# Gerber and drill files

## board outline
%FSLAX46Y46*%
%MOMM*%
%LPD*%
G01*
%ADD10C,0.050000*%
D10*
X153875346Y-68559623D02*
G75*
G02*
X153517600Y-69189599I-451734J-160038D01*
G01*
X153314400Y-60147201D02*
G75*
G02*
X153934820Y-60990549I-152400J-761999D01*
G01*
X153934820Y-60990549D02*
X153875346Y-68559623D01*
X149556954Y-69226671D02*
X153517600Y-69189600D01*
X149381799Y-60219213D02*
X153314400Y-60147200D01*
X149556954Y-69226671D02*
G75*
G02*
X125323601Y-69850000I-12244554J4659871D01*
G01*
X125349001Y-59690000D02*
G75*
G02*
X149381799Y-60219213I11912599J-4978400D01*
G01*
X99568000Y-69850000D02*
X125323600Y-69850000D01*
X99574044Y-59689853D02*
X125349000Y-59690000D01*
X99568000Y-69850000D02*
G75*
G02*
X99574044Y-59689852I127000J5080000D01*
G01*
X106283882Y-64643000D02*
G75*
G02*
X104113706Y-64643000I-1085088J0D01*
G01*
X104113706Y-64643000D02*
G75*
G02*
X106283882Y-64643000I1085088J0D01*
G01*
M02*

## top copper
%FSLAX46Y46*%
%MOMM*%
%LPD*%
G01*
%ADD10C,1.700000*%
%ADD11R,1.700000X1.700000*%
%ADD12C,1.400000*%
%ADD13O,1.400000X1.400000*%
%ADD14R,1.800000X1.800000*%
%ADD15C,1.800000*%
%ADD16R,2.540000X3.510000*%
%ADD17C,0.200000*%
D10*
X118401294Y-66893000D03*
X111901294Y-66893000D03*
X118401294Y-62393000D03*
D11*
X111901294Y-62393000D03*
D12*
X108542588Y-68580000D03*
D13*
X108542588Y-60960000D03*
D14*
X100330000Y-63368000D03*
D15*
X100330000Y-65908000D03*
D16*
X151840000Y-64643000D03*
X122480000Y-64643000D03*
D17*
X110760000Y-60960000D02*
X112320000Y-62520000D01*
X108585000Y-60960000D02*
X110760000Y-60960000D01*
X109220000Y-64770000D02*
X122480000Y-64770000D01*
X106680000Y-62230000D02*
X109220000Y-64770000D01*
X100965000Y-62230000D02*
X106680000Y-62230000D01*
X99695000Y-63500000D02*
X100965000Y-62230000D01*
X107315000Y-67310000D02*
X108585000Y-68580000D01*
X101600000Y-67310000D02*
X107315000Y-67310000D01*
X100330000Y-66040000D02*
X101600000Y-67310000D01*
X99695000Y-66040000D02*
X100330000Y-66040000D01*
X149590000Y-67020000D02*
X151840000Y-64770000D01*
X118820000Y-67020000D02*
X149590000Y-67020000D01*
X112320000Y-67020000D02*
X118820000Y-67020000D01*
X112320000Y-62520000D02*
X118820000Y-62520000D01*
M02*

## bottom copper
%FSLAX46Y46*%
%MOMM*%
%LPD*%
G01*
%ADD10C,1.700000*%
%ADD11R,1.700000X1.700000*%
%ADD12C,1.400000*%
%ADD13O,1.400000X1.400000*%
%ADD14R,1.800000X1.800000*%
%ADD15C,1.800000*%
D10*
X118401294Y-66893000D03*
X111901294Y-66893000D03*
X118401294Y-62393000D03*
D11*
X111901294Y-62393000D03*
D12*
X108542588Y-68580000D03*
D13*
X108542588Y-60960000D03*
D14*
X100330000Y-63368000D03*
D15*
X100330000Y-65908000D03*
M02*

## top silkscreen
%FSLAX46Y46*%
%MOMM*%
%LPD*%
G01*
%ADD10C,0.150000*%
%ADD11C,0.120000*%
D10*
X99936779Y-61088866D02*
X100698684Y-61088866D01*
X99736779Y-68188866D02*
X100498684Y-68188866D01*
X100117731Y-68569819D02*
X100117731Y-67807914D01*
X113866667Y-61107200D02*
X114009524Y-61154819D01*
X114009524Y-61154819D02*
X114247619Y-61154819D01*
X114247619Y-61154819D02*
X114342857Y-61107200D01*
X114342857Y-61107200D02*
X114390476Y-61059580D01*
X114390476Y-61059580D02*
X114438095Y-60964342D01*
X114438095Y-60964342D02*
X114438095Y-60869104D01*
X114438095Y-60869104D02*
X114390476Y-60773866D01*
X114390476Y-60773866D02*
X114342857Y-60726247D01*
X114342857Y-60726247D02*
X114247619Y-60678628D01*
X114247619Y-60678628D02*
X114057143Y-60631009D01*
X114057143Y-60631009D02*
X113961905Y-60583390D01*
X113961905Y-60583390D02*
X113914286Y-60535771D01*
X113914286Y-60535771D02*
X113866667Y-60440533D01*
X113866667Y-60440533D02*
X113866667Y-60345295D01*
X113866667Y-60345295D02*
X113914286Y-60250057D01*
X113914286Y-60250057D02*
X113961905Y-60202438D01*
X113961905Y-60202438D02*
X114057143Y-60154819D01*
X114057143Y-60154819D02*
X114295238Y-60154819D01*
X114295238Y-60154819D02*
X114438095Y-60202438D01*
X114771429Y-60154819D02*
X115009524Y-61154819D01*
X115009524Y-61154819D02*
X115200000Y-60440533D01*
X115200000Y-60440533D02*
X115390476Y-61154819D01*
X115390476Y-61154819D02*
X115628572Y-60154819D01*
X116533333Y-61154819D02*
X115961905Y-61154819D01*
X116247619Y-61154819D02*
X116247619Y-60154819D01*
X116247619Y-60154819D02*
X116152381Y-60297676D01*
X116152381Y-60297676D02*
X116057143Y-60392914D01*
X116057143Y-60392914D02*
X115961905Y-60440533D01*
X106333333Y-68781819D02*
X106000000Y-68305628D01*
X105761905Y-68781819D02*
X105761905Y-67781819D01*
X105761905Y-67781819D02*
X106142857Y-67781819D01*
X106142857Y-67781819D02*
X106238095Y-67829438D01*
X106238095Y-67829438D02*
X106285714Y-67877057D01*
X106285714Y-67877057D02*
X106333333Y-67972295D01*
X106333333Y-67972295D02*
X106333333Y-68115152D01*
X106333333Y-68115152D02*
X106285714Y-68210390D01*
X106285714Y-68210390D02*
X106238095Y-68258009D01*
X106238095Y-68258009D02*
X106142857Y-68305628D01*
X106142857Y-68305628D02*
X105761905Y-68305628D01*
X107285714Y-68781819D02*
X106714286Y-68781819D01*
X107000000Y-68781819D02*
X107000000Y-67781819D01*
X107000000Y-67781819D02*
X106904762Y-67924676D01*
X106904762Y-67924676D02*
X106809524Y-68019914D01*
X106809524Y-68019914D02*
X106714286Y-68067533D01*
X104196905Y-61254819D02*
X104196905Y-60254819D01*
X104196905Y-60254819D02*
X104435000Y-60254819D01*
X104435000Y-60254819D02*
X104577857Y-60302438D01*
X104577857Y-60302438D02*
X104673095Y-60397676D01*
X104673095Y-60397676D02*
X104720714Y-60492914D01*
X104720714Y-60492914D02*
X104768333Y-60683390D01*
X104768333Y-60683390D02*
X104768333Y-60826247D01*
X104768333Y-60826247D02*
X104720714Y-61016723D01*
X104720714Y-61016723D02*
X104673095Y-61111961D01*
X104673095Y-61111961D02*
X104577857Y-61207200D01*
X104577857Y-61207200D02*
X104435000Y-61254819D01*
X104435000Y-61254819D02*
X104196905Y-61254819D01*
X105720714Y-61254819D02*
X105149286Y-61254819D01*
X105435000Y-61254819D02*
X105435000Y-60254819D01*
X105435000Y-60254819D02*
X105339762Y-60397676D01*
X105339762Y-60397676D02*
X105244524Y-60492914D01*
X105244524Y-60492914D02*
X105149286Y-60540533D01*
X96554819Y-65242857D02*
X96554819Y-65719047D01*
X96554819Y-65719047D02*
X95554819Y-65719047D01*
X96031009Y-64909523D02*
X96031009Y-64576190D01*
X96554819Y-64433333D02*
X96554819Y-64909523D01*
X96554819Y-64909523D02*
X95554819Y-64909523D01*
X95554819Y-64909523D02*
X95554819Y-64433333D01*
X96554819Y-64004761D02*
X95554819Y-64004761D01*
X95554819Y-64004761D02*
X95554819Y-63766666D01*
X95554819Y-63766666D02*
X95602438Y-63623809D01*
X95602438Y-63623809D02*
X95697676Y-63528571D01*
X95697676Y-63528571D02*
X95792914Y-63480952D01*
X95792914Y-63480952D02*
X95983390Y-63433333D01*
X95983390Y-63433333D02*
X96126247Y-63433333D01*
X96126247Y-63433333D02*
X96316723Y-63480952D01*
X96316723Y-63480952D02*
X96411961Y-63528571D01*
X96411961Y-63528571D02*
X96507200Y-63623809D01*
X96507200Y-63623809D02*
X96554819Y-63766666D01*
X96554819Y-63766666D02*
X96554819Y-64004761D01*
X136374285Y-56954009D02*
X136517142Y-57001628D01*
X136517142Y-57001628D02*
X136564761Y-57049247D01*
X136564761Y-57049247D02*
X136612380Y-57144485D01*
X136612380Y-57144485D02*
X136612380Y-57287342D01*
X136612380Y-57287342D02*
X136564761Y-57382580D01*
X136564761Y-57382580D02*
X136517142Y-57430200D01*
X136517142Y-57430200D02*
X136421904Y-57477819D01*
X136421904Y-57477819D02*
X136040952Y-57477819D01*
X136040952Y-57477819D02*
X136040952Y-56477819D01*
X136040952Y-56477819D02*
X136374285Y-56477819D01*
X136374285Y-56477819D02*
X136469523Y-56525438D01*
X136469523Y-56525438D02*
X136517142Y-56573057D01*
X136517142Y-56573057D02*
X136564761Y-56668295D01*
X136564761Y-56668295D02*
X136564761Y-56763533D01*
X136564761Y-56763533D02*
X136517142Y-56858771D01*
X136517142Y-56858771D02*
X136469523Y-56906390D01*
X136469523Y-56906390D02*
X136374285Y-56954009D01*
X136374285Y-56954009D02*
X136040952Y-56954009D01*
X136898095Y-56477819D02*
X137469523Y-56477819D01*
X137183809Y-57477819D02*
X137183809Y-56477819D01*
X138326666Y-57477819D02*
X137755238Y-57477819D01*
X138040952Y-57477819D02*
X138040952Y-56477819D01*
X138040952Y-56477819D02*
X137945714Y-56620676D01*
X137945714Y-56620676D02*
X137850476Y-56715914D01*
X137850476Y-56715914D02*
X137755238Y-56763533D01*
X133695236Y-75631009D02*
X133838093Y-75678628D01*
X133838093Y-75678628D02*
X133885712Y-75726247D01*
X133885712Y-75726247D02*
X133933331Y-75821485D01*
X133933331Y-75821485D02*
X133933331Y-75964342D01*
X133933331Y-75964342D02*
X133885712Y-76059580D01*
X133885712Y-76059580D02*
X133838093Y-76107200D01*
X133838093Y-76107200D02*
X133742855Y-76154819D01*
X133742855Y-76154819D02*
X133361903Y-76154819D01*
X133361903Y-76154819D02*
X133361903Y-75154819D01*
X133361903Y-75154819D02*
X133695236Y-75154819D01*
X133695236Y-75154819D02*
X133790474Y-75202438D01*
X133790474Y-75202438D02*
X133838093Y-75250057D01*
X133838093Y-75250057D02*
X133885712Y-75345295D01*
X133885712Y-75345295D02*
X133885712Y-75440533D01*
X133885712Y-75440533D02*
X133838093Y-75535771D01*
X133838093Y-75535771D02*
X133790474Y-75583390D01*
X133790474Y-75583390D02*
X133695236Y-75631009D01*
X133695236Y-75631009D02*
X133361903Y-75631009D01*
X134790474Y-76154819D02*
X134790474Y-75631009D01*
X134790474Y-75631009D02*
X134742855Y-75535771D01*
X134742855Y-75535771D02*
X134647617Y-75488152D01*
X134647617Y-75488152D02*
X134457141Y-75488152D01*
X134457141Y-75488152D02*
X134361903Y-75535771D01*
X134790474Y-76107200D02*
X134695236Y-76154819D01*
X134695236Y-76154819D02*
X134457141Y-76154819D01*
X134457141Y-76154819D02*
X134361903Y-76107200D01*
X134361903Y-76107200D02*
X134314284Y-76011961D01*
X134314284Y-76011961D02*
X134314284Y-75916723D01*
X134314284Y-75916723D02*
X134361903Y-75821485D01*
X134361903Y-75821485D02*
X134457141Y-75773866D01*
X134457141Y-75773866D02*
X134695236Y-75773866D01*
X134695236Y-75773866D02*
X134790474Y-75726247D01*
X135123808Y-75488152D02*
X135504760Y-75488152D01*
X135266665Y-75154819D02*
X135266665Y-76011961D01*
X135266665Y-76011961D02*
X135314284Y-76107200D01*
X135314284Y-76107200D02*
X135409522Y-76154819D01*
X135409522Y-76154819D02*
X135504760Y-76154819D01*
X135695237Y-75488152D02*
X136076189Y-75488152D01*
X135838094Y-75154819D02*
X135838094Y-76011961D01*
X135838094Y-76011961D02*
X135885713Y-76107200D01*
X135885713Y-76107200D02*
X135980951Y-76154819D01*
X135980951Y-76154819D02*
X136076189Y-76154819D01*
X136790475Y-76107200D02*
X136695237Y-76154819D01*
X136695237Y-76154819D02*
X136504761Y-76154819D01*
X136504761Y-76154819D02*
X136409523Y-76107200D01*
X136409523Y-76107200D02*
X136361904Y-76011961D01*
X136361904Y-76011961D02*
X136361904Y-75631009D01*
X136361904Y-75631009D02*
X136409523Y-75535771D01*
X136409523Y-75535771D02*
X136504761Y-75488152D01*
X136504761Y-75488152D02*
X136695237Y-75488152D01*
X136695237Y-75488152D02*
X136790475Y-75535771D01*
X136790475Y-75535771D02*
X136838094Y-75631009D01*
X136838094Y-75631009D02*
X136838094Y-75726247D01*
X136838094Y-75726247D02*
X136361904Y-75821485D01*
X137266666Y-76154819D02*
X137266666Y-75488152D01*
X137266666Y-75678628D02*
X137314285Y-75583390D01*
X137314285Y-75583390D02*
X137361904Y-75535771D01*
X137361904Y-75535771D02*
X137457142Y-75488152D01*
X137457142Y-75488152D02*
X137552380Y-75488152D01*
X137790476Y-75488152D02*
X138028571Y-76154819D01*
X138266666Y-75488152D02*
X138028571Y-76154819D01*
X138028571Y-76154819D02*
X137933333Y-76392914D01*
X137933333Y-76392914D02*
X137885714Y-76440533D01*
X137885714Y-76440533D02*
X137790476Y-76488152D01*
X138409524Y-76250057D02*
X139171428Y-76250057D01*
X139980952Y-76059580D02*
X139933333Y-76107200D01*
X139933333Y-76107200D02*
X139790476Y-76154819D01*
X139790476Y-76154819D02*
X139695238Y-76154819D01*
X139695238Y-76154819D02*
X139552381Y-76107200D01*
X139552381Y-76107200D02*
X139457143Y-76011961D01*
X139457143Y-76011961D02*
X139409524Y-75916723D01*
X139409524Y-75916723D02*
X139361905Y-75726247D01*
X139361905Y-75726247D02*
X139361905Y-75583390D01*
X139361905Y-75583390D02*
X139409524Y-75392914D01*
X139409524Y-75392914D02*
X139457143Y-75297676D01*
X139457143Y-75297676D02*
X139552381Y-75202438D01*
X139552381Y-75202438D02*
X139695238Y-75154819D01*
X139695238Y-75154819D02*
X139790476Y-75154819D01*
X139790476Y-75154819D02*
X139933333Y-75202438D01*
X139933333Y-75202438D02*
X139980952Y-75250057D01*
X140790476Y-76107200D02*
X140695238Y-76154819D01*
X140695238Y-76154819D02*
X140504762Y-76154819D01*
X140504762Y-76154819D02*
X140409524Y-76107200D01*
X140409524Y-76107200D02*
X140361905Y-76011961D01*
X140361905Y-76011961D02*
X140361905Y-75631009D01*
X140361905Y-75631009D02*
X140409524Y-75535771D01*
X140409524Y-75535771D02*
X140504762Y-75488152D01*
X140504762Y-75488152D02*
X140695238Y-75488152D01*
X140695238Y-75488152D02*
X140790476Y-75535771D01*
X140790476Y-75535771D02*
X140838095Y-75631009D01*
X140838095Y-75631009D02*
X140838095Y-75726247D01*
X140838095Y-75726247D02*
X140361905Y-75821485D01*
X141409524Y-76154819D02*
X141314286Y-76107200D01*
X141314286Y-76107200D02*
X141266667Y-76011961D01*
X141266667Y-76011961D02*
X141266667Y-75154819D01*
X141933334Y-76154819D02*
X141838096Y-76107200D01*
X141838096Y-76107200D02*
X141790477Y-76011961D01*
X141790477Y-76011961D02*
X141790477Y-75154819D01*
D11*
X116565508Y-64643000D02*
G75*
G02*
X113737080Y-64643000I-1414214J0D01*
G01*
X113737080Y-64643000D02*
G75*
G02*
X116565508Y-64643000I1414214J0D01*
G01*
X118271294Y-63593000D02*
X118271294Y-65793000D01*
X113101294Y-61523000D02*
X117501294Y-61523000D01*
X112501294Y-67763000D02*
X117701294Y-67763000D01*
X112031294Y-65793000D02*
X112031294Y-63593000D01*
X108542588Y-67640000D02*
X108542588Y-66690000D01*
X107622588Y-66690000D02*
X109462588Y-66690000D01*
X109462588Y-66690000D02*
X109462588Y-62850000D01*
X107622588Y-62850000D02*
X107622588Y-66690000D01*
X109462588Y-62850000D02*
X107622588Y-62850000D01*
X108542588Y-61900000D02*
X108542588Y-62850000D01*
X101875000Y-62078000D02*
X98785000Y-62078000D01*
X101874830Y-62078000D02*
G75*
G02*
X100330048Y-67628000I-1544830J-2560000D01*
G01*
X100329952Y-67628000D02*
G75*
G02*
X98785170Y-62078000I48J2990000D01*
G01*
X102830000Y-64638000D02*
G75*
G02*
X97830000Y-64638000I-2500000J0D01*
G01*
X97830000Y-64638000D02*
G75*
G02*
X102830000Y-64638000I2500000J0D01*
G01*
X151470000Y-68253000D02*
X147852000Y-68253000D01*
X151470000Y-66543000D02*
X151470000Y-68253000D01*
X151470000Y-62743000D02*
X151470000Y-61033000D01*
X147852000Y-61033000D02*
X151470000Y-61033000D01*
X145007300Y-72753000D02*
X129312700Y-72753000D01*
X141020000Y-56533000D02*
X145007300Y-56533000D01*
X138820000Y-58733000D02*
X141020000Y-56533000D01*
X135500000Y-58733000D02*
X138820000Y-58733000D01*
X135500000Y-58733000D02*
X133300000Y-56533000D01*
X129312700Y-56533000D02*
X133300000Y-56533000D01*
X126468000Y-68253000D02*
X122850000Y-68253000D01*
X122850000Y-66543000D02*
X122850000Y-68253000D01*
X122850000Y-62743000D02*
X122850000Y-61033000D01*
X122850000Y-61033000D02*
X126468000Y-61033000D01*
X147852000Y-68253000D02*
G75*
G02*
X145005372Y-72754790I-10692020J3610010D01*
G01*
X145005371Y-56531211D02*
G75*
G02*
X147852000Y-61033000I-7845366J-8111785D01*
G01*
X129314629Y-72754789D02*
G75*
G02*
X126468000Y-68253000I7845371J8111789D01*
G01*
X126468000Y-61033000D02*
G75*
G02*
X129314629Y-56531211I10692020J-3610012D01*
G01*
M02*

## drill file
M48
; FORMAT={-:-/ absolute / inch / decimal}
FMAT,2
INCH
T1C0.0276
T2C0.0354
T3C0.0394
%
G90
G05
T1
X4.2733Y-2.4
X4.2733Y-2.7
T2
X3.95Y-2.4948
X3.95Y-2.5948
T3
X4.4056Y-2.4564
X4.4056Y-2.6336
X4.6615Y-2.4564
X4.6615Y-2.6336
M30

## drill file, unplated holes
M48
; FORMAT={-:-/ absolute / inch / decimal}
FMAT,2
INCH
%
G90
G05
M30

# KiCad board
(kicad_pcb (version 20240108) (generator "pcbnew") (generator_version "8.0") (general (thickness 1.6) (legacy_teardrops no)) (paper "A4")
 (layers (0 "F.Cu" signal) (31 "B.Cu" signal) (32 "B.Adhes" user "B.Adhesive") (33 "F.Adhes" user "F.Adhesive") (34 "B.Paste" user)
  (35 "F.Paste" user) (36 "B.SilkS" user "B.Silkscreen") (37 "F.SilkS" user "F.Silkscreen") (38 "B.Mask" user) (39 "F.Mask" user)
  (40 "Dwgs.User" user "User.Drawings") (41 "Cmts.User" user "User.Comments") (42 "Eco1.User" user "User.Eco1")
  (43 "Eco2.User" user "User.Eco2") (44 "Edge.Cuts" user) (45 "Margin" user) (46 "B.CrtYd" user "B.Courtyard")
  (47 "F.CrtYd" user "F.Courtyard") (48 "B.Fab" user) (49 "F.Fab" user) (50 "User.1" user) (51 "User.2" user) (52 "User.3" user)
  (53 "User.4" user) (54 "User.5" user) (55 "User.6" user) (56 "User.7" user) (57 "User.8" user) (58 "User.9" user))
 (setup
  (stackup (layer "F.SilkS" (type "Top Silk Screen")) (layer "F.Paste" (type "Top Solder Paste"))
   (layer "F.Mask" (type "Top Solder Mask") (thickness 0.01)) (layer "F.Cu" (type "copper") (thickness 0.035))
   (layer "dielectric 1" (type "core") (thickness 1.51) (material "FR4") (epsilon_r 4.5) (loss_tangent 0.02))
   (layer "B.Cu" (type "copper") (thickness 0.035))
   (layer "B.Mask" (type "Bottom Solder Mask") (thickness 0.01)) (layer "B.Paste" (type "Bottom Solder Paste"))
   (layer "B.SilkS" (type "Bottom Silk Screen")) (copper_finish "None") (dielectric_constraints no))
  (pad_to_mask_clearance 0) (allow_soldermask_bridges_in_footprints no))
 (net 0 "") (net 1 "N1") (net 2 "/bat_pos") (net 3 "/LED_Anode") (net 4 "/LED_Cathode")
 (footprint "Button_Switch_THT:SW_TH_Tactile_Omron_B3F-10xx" (layer "F.Cu") (at 111.901294 62.393)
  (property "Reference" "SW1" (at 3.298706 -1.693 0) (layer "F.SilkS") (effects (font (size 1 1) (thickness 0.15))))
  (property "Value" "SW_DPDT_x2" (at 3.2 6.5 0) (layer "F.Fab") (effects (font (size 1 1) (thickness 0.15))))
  (fp_line (start 0.13 3.4) (end 0.13 1.2) (stroke (width 0.12) (type solid)) (layer "F.SilkS"))
  (fp_line (start 0.6 5.37) (end 5.8 5.37) (stroke (width 0.12) (type solid)) (layer "F.SilkS"))
  (fp_line (start 1.2 -0.87) (end 5.6 -0.87) (stroke (width 0.12) (type solid)) (layer "F.SilkS"))
  (fp_line (start 6.37 1.2) (end 6.37 3.4) (stroke (width 0.12) (type solid)) (layer "F.SilkS"))
  (fp_circle (center 3.25 2.25) (end 4.25 3.25) (stroke (width 0.12) (type solid)) (fill none) (layer "F.SilkS"))
  (pad "1" thru_hole rect (at 0 0) (size 1.7 1.7) (drill 1) (layers "*.Cu" "*.Mask") (remove_unused_layers no) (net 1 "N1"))
  (pad "1" thru_hole circle (at 6.5 0) (size 1.7 1.7) (drill 1) (layers "*.Cu" "*.Mask") (remove_unused_layers no) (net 1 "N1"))
  (pad "2" thru_hole circle (at 0 4.5) (size 1.7 1.7) (drill 1) (layers "*.Cu" "*.Mask") (remove_unused_layers no) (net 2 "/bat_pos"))
  (pad "2" thru_hole circle (at 6.5 4.5) (size 1.7 1.7) (drill 1) (layers "*.Cu" "*.Mask") (remove_unused_layers no) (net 2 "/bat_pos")))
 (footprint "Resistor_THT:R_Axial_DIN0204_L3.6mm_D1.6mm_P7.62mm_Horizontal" (layer "F.Cu") (at 108.542588 68.58 90)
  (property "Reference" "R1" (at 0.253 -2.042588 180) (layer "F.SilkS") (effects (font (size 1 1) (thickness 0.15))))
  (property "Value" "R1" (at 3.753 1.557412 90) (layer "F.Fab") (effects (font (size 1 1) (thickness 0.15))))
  (fp_line (start 5.73 -0.92) (end 1.89 -0.92) (stroke (width 0.12) (type solid)) (layer "F.SilkS"))
  (fp_line (start 1.89 -0.92) (end 1.89 0.92) (stroke (width 0.12) (type solid)) (layer "F.SilkS"))
  (fp_line (start 6.68 0) (end 5.73 0) (stroke (width 0.12) (type solid)) (layer "F.SilkS"))
  (fp_line (start 0.94 0) (end 1.89 0) (stroke (width 0.12) (type solid)) (layer "F.SilkS"))
  (fp_line (start 5.73 0.92) (end 5.73 -0.92) (stroke (width 0.12) (type solid)) (layer "F.SilkS"))
  (fp_line (start 1.89 0.92) (end 5.73 0.92) (stroke (width 0.12) (type solid)) (layer "F.SilkS"))
  (pad "1" thru_hole circle (at 0 0 90) (size 1.4 1.4) (drill 0.7) (layers "*.Cu" "*.Mask") (remove_unused_layers no) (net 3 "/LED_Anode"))
  (pad "2" thru_hole oval (at 7.62 0 90) (size 1.4 1.4) (drill 0.7) (layers "*.Cu" "*.Mask") (remove_unused_layers no) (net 1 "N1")))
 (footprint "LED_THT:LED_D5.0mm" (layer "F.Cu") (at 100.33 63.368 -90)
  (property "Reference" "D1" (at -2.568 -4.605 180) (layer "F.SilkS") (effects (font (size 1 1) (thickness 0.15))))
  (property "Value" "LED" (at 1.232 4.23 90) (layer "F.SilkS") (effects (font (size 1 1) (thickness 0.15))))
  (fp_line (start -1.29 -1.545) (end -1.29 1.545) (stroke (width 0.12) (type solid)) (layer "F.SilkS"))
  (fp_arc (start 4.26 0.000048) (mid 2.071756 2.880501) (end -1.29 1.54483) (stroke (width 0.12) (type solid)) (layer "F.SilkS"))
  (fp_arc (start -1.29 -1.54483) (mid 2.071756 -2.880501) (end 4.26 -0.000048) (stroke (width 0.12) (type solid)) (layer "F.SilkS"))
  (fp_circle (center 1.27 0) (end 3.77 0) (stroke (width 0.12) (type solid)) (fill none) (layer "F.SilkS"))
  (pad "1" thru_hole rect (at 0 0 270) (size 1.8 1.8) (drill 0.9) (layers "*.Cu" "*.Mask") (remove_unused_layers no) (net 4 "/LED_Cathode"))
  (pad "2" thru_hole circle (at 2.54 0 270) (size 1.8 1.8) (drill 0.9) (layers "*.Cu" "*.Mask") (remove_unused_layers no)
   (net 3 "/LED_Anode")))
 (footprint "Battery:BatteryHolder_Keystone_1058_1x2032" (layer "F.Cu") (at 137.16 64.643 180)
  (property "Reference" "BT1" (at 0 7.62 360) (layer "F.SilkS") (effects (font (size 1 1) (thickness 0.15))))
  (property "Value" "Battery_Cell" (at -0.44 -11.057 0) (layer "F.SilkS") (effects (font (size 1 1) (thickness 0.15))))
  (fp_line (start 14.31 3.61) (end 10.692 3.61) (stroke (width 0.12) (type solid)) (layer "F.SilkS"))
  (fp_line (start 14.31 1.9) (end 14.31 3.61) (stroke (width 0.12) (type solid)) (layer "F.SilkS"))
  (fp_line (start 14.31 -1.9) (end 14.31 -3.61) (stroke (width 0.12) (type solid)) (layer "F.SilkS"))
  (fp_line (start 10.692 -3.61) (end 14.31 -3.61) (stroke (width 0.12) (type solid)) (layer "F.SilkS"))
  (fp_line (start 7.8473 8.11) (end 3.86 8.11) (stroke (width 0.12) (type solid)) (layer "F.SilkS"))
  (fp_line (start 1.66 5.91) (end 3.86 8.11) (stroke (width 0.12) (type solid)) (layer "F.SilkS"))
  (fp_line (start 1.66 5.91) (end -1.66 5.91) (stroke (width 0.12) (type solid)) (layer "F.SilkS"))
  (fp_line (start -1.66 5.91) (end -3.86 8.11) (stroke (width 0.12) (type solid)) (layer "F.SilkS"))
  (fp_line (start -3.86 8.11) (end -7.8473 8.11) (stroke (width 0.12) (type solid)) (layer "F.SilkS"))
  (fp_line (start -7.8473 -8.11) (end 7.8473 -8.11) (stroke (width 0.12) (type solid)) (layer "F.SilkS"))
  (fp_line (start -10.692 3.61) (end -14.31 3.61) (stroke (width 0.12) (type solid)) (layer "F.SilkS"))
  (fp_line (start -14.31 1.9) (end -14.31 3.61) (stroke (width 0.12) (type solid)) (layer "F.SilkS"))
  (fp_line (start -14.31 -1.9) (end -14.31 -3.61) (stroke (width 0.12) (type solid)) (layer "F.SilkS"))
  (fp_line (start -14.31 -3.61) (end -10.692 -3.61) (stroke (width 0.12) (type solid)) (layer "F.SilkS"))
  (fp_arc (start 10.692 3.61) (mid 9.538084 6.031244) (end 7.845371 8.111789) (stroke (width 0.12) (type solid)) (layer "F.SilkS"))
  (fp_arc (start 7.845371 -8.111789) (mid 9.538085 -6.031244) (end 10.692 -3.61) (stroke (width 0.12) (type solid)) (layer "F.SilkS"))
  (fp_arc (start -7.845371 8.111789) (mid -9.538085 6.031244) (end -10.692 3.61) (stroke (width 0.12) (type solid)) (layer "F.SilkS"))
  (fp_arc (start -10.692 -3.61) (mid -9.538084 -6.031244) (end -7.845371 -8.111789) (stroke (width 0.12) (type solid)) (layer "F.SilkS"))
  (pad "1" smd rect (at -14.68 0 180) (size 2.54 3.51) (layers "F.Cu" "F.Paste" "F.Mask") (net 2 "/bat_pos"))
  (pad "2" smd rect (at 14.68 0 180) (size 2.54 3.51) (layers "F.Cu" "F.Paste" "F.Mask") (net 4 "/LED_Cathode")))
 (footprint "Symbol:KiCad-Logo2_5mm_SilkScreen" (layer "B.Cu") (at 136.8806 62.0268 180)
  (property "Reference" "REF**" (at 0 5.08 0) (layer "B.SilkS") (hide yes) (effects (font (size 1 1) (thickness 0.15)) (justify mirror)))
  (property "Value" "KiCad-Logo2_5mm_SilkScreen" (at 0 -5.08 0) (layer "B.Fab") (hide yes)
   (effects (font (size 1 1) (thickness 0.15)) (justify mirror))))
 (gr_line (start 99.568 69.85) (end 125.3236 69.85) (locked yes) (stroke (width 0.05) (type default)) (layer "Edge.Cuts"))
 (gr_line (start 99.574044 59.689853) (end 125.349 59.69) (locked yes) (stroke (width 0.05) (type default)) (layer "Edge.Cuts"))
 (gr_circle (center 105.198794 64.643) (end 104.182794 65.024) (stroke (width 0.05) (type default)) (fill none) (layer "Edge.Cuts"))
 (gr_arc (start 153.875346 68.559623) (mid 153.84035 68.956315) (end 153.5176 69.189599) (locked yes) (stroke (width 0.05) (type default))
  (layer "Edge.Cuts"))
 (gr_line (start 149.556954 69.226671) (end 153.5176 69.1896) (locked yes) (stroke (width 0.05) (type default)) (layer "Edge.Cuts"))
 (gr_arc (start 149.556954 69.226671) (mid 137.649279 77.663747) (end 125.323601 69.85) (locked yes) (stroke (width 0.05) (type default))
  (layer "Edge.Cuts"))
 (gr_line (start 153.93482 60.990549) (end 153.875346 68.559623) (locked yes) (stroke (width 0.05) (type default)) (layer "Edge.Cuts"))
 (gr_line (start 149.381799 60.219213) (end 153.3144 60.1472) (locked yes) (stroke (width 0.05) (type default)) (layer "Edge.Cuts"))
 (gr_arc (start 153.3144 60.147201) (mid 153.787953 60.44871) (end 153.93482 60.990549) (locked yes) (stroke (width 0.05) (type default))
  (layer "Edge.Cuts"))
 (gr_arc (start 125.349001 59.69) (mid 137.545838 51.760507) (end 149.381799 60.219213) (locked yes) (stroke (width 0.05) (type default))
  (layer "Edge.Cuts"))
 (gr_arc (start 99.568 69.85) (mid 94.613414 64.766977) (end 99.574044 59.689853) (locked yes) (stroke (width 0.05) (type default))
  (layer "Edge.Cuts"))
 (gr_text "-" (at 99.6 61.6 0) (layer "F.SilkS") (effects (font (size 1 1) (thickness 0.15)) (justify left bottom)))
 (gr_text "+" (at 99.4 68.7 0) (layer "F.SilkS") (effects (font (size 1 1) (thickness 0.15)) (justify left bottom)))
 (segment (start 109.22 64.77) (end 122.48 64.77) (width 0.2) (layer "F.Cu") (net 4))
 (segment (start 99.695 63.5) (end 100.965 62.23) (width 0.2) (layer "F.Cu") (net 4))
 (segment (start 106.68 62.23) (end 109.22 64.77) (width 0.2) (layer "F.Cu") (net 4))
 (segment (start 100.965 62.23) (end 106.68 62.23) (width 0.2) (layer "F.Cu") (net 4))
 (segment (start 118.82 67.02) (end 149.59 67.02) (width 0.2) (layer "F.Cu") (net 2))
 (segment (start 112.32 67.02) (end 118.82 67.02) (width 0.2) (layer "F.Cu") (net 2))
 (segment (start 149.59 67.02) (end 151.84 64.77) (width 0.2) (layer "F.Cu") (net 2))
 (segment (start 100.33 66.04) (end 101.6 67.31) (width 0.2) (layer "F.Cu") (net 3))
 (segment (start 101.6 67.31) (end 107.315 67.31) (width 0.2) (layer "F.Cu") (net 3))
 (segment (start 99.695 66.04) (end 100.33 66.04) (width 0.2) (layer "F.Cu") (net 3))
 (segment (start 107.315 67.31) (end 108.585 68.58) (width 0.2) (layer "F.Cu") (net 3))
 (segment (start 112.32 62.52) (end 118.82 62.52) (width 0.2) (layer "F.Cu") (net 1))
 (segment (start 110.76 60.96) (end 112.32 62.52) (width 0.2) (layer "F.Cu") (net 1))
 (segment (start 108.585 60.96) (end 110.76 60.96) (width 0.2) (layer "F.Cu") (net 1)))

